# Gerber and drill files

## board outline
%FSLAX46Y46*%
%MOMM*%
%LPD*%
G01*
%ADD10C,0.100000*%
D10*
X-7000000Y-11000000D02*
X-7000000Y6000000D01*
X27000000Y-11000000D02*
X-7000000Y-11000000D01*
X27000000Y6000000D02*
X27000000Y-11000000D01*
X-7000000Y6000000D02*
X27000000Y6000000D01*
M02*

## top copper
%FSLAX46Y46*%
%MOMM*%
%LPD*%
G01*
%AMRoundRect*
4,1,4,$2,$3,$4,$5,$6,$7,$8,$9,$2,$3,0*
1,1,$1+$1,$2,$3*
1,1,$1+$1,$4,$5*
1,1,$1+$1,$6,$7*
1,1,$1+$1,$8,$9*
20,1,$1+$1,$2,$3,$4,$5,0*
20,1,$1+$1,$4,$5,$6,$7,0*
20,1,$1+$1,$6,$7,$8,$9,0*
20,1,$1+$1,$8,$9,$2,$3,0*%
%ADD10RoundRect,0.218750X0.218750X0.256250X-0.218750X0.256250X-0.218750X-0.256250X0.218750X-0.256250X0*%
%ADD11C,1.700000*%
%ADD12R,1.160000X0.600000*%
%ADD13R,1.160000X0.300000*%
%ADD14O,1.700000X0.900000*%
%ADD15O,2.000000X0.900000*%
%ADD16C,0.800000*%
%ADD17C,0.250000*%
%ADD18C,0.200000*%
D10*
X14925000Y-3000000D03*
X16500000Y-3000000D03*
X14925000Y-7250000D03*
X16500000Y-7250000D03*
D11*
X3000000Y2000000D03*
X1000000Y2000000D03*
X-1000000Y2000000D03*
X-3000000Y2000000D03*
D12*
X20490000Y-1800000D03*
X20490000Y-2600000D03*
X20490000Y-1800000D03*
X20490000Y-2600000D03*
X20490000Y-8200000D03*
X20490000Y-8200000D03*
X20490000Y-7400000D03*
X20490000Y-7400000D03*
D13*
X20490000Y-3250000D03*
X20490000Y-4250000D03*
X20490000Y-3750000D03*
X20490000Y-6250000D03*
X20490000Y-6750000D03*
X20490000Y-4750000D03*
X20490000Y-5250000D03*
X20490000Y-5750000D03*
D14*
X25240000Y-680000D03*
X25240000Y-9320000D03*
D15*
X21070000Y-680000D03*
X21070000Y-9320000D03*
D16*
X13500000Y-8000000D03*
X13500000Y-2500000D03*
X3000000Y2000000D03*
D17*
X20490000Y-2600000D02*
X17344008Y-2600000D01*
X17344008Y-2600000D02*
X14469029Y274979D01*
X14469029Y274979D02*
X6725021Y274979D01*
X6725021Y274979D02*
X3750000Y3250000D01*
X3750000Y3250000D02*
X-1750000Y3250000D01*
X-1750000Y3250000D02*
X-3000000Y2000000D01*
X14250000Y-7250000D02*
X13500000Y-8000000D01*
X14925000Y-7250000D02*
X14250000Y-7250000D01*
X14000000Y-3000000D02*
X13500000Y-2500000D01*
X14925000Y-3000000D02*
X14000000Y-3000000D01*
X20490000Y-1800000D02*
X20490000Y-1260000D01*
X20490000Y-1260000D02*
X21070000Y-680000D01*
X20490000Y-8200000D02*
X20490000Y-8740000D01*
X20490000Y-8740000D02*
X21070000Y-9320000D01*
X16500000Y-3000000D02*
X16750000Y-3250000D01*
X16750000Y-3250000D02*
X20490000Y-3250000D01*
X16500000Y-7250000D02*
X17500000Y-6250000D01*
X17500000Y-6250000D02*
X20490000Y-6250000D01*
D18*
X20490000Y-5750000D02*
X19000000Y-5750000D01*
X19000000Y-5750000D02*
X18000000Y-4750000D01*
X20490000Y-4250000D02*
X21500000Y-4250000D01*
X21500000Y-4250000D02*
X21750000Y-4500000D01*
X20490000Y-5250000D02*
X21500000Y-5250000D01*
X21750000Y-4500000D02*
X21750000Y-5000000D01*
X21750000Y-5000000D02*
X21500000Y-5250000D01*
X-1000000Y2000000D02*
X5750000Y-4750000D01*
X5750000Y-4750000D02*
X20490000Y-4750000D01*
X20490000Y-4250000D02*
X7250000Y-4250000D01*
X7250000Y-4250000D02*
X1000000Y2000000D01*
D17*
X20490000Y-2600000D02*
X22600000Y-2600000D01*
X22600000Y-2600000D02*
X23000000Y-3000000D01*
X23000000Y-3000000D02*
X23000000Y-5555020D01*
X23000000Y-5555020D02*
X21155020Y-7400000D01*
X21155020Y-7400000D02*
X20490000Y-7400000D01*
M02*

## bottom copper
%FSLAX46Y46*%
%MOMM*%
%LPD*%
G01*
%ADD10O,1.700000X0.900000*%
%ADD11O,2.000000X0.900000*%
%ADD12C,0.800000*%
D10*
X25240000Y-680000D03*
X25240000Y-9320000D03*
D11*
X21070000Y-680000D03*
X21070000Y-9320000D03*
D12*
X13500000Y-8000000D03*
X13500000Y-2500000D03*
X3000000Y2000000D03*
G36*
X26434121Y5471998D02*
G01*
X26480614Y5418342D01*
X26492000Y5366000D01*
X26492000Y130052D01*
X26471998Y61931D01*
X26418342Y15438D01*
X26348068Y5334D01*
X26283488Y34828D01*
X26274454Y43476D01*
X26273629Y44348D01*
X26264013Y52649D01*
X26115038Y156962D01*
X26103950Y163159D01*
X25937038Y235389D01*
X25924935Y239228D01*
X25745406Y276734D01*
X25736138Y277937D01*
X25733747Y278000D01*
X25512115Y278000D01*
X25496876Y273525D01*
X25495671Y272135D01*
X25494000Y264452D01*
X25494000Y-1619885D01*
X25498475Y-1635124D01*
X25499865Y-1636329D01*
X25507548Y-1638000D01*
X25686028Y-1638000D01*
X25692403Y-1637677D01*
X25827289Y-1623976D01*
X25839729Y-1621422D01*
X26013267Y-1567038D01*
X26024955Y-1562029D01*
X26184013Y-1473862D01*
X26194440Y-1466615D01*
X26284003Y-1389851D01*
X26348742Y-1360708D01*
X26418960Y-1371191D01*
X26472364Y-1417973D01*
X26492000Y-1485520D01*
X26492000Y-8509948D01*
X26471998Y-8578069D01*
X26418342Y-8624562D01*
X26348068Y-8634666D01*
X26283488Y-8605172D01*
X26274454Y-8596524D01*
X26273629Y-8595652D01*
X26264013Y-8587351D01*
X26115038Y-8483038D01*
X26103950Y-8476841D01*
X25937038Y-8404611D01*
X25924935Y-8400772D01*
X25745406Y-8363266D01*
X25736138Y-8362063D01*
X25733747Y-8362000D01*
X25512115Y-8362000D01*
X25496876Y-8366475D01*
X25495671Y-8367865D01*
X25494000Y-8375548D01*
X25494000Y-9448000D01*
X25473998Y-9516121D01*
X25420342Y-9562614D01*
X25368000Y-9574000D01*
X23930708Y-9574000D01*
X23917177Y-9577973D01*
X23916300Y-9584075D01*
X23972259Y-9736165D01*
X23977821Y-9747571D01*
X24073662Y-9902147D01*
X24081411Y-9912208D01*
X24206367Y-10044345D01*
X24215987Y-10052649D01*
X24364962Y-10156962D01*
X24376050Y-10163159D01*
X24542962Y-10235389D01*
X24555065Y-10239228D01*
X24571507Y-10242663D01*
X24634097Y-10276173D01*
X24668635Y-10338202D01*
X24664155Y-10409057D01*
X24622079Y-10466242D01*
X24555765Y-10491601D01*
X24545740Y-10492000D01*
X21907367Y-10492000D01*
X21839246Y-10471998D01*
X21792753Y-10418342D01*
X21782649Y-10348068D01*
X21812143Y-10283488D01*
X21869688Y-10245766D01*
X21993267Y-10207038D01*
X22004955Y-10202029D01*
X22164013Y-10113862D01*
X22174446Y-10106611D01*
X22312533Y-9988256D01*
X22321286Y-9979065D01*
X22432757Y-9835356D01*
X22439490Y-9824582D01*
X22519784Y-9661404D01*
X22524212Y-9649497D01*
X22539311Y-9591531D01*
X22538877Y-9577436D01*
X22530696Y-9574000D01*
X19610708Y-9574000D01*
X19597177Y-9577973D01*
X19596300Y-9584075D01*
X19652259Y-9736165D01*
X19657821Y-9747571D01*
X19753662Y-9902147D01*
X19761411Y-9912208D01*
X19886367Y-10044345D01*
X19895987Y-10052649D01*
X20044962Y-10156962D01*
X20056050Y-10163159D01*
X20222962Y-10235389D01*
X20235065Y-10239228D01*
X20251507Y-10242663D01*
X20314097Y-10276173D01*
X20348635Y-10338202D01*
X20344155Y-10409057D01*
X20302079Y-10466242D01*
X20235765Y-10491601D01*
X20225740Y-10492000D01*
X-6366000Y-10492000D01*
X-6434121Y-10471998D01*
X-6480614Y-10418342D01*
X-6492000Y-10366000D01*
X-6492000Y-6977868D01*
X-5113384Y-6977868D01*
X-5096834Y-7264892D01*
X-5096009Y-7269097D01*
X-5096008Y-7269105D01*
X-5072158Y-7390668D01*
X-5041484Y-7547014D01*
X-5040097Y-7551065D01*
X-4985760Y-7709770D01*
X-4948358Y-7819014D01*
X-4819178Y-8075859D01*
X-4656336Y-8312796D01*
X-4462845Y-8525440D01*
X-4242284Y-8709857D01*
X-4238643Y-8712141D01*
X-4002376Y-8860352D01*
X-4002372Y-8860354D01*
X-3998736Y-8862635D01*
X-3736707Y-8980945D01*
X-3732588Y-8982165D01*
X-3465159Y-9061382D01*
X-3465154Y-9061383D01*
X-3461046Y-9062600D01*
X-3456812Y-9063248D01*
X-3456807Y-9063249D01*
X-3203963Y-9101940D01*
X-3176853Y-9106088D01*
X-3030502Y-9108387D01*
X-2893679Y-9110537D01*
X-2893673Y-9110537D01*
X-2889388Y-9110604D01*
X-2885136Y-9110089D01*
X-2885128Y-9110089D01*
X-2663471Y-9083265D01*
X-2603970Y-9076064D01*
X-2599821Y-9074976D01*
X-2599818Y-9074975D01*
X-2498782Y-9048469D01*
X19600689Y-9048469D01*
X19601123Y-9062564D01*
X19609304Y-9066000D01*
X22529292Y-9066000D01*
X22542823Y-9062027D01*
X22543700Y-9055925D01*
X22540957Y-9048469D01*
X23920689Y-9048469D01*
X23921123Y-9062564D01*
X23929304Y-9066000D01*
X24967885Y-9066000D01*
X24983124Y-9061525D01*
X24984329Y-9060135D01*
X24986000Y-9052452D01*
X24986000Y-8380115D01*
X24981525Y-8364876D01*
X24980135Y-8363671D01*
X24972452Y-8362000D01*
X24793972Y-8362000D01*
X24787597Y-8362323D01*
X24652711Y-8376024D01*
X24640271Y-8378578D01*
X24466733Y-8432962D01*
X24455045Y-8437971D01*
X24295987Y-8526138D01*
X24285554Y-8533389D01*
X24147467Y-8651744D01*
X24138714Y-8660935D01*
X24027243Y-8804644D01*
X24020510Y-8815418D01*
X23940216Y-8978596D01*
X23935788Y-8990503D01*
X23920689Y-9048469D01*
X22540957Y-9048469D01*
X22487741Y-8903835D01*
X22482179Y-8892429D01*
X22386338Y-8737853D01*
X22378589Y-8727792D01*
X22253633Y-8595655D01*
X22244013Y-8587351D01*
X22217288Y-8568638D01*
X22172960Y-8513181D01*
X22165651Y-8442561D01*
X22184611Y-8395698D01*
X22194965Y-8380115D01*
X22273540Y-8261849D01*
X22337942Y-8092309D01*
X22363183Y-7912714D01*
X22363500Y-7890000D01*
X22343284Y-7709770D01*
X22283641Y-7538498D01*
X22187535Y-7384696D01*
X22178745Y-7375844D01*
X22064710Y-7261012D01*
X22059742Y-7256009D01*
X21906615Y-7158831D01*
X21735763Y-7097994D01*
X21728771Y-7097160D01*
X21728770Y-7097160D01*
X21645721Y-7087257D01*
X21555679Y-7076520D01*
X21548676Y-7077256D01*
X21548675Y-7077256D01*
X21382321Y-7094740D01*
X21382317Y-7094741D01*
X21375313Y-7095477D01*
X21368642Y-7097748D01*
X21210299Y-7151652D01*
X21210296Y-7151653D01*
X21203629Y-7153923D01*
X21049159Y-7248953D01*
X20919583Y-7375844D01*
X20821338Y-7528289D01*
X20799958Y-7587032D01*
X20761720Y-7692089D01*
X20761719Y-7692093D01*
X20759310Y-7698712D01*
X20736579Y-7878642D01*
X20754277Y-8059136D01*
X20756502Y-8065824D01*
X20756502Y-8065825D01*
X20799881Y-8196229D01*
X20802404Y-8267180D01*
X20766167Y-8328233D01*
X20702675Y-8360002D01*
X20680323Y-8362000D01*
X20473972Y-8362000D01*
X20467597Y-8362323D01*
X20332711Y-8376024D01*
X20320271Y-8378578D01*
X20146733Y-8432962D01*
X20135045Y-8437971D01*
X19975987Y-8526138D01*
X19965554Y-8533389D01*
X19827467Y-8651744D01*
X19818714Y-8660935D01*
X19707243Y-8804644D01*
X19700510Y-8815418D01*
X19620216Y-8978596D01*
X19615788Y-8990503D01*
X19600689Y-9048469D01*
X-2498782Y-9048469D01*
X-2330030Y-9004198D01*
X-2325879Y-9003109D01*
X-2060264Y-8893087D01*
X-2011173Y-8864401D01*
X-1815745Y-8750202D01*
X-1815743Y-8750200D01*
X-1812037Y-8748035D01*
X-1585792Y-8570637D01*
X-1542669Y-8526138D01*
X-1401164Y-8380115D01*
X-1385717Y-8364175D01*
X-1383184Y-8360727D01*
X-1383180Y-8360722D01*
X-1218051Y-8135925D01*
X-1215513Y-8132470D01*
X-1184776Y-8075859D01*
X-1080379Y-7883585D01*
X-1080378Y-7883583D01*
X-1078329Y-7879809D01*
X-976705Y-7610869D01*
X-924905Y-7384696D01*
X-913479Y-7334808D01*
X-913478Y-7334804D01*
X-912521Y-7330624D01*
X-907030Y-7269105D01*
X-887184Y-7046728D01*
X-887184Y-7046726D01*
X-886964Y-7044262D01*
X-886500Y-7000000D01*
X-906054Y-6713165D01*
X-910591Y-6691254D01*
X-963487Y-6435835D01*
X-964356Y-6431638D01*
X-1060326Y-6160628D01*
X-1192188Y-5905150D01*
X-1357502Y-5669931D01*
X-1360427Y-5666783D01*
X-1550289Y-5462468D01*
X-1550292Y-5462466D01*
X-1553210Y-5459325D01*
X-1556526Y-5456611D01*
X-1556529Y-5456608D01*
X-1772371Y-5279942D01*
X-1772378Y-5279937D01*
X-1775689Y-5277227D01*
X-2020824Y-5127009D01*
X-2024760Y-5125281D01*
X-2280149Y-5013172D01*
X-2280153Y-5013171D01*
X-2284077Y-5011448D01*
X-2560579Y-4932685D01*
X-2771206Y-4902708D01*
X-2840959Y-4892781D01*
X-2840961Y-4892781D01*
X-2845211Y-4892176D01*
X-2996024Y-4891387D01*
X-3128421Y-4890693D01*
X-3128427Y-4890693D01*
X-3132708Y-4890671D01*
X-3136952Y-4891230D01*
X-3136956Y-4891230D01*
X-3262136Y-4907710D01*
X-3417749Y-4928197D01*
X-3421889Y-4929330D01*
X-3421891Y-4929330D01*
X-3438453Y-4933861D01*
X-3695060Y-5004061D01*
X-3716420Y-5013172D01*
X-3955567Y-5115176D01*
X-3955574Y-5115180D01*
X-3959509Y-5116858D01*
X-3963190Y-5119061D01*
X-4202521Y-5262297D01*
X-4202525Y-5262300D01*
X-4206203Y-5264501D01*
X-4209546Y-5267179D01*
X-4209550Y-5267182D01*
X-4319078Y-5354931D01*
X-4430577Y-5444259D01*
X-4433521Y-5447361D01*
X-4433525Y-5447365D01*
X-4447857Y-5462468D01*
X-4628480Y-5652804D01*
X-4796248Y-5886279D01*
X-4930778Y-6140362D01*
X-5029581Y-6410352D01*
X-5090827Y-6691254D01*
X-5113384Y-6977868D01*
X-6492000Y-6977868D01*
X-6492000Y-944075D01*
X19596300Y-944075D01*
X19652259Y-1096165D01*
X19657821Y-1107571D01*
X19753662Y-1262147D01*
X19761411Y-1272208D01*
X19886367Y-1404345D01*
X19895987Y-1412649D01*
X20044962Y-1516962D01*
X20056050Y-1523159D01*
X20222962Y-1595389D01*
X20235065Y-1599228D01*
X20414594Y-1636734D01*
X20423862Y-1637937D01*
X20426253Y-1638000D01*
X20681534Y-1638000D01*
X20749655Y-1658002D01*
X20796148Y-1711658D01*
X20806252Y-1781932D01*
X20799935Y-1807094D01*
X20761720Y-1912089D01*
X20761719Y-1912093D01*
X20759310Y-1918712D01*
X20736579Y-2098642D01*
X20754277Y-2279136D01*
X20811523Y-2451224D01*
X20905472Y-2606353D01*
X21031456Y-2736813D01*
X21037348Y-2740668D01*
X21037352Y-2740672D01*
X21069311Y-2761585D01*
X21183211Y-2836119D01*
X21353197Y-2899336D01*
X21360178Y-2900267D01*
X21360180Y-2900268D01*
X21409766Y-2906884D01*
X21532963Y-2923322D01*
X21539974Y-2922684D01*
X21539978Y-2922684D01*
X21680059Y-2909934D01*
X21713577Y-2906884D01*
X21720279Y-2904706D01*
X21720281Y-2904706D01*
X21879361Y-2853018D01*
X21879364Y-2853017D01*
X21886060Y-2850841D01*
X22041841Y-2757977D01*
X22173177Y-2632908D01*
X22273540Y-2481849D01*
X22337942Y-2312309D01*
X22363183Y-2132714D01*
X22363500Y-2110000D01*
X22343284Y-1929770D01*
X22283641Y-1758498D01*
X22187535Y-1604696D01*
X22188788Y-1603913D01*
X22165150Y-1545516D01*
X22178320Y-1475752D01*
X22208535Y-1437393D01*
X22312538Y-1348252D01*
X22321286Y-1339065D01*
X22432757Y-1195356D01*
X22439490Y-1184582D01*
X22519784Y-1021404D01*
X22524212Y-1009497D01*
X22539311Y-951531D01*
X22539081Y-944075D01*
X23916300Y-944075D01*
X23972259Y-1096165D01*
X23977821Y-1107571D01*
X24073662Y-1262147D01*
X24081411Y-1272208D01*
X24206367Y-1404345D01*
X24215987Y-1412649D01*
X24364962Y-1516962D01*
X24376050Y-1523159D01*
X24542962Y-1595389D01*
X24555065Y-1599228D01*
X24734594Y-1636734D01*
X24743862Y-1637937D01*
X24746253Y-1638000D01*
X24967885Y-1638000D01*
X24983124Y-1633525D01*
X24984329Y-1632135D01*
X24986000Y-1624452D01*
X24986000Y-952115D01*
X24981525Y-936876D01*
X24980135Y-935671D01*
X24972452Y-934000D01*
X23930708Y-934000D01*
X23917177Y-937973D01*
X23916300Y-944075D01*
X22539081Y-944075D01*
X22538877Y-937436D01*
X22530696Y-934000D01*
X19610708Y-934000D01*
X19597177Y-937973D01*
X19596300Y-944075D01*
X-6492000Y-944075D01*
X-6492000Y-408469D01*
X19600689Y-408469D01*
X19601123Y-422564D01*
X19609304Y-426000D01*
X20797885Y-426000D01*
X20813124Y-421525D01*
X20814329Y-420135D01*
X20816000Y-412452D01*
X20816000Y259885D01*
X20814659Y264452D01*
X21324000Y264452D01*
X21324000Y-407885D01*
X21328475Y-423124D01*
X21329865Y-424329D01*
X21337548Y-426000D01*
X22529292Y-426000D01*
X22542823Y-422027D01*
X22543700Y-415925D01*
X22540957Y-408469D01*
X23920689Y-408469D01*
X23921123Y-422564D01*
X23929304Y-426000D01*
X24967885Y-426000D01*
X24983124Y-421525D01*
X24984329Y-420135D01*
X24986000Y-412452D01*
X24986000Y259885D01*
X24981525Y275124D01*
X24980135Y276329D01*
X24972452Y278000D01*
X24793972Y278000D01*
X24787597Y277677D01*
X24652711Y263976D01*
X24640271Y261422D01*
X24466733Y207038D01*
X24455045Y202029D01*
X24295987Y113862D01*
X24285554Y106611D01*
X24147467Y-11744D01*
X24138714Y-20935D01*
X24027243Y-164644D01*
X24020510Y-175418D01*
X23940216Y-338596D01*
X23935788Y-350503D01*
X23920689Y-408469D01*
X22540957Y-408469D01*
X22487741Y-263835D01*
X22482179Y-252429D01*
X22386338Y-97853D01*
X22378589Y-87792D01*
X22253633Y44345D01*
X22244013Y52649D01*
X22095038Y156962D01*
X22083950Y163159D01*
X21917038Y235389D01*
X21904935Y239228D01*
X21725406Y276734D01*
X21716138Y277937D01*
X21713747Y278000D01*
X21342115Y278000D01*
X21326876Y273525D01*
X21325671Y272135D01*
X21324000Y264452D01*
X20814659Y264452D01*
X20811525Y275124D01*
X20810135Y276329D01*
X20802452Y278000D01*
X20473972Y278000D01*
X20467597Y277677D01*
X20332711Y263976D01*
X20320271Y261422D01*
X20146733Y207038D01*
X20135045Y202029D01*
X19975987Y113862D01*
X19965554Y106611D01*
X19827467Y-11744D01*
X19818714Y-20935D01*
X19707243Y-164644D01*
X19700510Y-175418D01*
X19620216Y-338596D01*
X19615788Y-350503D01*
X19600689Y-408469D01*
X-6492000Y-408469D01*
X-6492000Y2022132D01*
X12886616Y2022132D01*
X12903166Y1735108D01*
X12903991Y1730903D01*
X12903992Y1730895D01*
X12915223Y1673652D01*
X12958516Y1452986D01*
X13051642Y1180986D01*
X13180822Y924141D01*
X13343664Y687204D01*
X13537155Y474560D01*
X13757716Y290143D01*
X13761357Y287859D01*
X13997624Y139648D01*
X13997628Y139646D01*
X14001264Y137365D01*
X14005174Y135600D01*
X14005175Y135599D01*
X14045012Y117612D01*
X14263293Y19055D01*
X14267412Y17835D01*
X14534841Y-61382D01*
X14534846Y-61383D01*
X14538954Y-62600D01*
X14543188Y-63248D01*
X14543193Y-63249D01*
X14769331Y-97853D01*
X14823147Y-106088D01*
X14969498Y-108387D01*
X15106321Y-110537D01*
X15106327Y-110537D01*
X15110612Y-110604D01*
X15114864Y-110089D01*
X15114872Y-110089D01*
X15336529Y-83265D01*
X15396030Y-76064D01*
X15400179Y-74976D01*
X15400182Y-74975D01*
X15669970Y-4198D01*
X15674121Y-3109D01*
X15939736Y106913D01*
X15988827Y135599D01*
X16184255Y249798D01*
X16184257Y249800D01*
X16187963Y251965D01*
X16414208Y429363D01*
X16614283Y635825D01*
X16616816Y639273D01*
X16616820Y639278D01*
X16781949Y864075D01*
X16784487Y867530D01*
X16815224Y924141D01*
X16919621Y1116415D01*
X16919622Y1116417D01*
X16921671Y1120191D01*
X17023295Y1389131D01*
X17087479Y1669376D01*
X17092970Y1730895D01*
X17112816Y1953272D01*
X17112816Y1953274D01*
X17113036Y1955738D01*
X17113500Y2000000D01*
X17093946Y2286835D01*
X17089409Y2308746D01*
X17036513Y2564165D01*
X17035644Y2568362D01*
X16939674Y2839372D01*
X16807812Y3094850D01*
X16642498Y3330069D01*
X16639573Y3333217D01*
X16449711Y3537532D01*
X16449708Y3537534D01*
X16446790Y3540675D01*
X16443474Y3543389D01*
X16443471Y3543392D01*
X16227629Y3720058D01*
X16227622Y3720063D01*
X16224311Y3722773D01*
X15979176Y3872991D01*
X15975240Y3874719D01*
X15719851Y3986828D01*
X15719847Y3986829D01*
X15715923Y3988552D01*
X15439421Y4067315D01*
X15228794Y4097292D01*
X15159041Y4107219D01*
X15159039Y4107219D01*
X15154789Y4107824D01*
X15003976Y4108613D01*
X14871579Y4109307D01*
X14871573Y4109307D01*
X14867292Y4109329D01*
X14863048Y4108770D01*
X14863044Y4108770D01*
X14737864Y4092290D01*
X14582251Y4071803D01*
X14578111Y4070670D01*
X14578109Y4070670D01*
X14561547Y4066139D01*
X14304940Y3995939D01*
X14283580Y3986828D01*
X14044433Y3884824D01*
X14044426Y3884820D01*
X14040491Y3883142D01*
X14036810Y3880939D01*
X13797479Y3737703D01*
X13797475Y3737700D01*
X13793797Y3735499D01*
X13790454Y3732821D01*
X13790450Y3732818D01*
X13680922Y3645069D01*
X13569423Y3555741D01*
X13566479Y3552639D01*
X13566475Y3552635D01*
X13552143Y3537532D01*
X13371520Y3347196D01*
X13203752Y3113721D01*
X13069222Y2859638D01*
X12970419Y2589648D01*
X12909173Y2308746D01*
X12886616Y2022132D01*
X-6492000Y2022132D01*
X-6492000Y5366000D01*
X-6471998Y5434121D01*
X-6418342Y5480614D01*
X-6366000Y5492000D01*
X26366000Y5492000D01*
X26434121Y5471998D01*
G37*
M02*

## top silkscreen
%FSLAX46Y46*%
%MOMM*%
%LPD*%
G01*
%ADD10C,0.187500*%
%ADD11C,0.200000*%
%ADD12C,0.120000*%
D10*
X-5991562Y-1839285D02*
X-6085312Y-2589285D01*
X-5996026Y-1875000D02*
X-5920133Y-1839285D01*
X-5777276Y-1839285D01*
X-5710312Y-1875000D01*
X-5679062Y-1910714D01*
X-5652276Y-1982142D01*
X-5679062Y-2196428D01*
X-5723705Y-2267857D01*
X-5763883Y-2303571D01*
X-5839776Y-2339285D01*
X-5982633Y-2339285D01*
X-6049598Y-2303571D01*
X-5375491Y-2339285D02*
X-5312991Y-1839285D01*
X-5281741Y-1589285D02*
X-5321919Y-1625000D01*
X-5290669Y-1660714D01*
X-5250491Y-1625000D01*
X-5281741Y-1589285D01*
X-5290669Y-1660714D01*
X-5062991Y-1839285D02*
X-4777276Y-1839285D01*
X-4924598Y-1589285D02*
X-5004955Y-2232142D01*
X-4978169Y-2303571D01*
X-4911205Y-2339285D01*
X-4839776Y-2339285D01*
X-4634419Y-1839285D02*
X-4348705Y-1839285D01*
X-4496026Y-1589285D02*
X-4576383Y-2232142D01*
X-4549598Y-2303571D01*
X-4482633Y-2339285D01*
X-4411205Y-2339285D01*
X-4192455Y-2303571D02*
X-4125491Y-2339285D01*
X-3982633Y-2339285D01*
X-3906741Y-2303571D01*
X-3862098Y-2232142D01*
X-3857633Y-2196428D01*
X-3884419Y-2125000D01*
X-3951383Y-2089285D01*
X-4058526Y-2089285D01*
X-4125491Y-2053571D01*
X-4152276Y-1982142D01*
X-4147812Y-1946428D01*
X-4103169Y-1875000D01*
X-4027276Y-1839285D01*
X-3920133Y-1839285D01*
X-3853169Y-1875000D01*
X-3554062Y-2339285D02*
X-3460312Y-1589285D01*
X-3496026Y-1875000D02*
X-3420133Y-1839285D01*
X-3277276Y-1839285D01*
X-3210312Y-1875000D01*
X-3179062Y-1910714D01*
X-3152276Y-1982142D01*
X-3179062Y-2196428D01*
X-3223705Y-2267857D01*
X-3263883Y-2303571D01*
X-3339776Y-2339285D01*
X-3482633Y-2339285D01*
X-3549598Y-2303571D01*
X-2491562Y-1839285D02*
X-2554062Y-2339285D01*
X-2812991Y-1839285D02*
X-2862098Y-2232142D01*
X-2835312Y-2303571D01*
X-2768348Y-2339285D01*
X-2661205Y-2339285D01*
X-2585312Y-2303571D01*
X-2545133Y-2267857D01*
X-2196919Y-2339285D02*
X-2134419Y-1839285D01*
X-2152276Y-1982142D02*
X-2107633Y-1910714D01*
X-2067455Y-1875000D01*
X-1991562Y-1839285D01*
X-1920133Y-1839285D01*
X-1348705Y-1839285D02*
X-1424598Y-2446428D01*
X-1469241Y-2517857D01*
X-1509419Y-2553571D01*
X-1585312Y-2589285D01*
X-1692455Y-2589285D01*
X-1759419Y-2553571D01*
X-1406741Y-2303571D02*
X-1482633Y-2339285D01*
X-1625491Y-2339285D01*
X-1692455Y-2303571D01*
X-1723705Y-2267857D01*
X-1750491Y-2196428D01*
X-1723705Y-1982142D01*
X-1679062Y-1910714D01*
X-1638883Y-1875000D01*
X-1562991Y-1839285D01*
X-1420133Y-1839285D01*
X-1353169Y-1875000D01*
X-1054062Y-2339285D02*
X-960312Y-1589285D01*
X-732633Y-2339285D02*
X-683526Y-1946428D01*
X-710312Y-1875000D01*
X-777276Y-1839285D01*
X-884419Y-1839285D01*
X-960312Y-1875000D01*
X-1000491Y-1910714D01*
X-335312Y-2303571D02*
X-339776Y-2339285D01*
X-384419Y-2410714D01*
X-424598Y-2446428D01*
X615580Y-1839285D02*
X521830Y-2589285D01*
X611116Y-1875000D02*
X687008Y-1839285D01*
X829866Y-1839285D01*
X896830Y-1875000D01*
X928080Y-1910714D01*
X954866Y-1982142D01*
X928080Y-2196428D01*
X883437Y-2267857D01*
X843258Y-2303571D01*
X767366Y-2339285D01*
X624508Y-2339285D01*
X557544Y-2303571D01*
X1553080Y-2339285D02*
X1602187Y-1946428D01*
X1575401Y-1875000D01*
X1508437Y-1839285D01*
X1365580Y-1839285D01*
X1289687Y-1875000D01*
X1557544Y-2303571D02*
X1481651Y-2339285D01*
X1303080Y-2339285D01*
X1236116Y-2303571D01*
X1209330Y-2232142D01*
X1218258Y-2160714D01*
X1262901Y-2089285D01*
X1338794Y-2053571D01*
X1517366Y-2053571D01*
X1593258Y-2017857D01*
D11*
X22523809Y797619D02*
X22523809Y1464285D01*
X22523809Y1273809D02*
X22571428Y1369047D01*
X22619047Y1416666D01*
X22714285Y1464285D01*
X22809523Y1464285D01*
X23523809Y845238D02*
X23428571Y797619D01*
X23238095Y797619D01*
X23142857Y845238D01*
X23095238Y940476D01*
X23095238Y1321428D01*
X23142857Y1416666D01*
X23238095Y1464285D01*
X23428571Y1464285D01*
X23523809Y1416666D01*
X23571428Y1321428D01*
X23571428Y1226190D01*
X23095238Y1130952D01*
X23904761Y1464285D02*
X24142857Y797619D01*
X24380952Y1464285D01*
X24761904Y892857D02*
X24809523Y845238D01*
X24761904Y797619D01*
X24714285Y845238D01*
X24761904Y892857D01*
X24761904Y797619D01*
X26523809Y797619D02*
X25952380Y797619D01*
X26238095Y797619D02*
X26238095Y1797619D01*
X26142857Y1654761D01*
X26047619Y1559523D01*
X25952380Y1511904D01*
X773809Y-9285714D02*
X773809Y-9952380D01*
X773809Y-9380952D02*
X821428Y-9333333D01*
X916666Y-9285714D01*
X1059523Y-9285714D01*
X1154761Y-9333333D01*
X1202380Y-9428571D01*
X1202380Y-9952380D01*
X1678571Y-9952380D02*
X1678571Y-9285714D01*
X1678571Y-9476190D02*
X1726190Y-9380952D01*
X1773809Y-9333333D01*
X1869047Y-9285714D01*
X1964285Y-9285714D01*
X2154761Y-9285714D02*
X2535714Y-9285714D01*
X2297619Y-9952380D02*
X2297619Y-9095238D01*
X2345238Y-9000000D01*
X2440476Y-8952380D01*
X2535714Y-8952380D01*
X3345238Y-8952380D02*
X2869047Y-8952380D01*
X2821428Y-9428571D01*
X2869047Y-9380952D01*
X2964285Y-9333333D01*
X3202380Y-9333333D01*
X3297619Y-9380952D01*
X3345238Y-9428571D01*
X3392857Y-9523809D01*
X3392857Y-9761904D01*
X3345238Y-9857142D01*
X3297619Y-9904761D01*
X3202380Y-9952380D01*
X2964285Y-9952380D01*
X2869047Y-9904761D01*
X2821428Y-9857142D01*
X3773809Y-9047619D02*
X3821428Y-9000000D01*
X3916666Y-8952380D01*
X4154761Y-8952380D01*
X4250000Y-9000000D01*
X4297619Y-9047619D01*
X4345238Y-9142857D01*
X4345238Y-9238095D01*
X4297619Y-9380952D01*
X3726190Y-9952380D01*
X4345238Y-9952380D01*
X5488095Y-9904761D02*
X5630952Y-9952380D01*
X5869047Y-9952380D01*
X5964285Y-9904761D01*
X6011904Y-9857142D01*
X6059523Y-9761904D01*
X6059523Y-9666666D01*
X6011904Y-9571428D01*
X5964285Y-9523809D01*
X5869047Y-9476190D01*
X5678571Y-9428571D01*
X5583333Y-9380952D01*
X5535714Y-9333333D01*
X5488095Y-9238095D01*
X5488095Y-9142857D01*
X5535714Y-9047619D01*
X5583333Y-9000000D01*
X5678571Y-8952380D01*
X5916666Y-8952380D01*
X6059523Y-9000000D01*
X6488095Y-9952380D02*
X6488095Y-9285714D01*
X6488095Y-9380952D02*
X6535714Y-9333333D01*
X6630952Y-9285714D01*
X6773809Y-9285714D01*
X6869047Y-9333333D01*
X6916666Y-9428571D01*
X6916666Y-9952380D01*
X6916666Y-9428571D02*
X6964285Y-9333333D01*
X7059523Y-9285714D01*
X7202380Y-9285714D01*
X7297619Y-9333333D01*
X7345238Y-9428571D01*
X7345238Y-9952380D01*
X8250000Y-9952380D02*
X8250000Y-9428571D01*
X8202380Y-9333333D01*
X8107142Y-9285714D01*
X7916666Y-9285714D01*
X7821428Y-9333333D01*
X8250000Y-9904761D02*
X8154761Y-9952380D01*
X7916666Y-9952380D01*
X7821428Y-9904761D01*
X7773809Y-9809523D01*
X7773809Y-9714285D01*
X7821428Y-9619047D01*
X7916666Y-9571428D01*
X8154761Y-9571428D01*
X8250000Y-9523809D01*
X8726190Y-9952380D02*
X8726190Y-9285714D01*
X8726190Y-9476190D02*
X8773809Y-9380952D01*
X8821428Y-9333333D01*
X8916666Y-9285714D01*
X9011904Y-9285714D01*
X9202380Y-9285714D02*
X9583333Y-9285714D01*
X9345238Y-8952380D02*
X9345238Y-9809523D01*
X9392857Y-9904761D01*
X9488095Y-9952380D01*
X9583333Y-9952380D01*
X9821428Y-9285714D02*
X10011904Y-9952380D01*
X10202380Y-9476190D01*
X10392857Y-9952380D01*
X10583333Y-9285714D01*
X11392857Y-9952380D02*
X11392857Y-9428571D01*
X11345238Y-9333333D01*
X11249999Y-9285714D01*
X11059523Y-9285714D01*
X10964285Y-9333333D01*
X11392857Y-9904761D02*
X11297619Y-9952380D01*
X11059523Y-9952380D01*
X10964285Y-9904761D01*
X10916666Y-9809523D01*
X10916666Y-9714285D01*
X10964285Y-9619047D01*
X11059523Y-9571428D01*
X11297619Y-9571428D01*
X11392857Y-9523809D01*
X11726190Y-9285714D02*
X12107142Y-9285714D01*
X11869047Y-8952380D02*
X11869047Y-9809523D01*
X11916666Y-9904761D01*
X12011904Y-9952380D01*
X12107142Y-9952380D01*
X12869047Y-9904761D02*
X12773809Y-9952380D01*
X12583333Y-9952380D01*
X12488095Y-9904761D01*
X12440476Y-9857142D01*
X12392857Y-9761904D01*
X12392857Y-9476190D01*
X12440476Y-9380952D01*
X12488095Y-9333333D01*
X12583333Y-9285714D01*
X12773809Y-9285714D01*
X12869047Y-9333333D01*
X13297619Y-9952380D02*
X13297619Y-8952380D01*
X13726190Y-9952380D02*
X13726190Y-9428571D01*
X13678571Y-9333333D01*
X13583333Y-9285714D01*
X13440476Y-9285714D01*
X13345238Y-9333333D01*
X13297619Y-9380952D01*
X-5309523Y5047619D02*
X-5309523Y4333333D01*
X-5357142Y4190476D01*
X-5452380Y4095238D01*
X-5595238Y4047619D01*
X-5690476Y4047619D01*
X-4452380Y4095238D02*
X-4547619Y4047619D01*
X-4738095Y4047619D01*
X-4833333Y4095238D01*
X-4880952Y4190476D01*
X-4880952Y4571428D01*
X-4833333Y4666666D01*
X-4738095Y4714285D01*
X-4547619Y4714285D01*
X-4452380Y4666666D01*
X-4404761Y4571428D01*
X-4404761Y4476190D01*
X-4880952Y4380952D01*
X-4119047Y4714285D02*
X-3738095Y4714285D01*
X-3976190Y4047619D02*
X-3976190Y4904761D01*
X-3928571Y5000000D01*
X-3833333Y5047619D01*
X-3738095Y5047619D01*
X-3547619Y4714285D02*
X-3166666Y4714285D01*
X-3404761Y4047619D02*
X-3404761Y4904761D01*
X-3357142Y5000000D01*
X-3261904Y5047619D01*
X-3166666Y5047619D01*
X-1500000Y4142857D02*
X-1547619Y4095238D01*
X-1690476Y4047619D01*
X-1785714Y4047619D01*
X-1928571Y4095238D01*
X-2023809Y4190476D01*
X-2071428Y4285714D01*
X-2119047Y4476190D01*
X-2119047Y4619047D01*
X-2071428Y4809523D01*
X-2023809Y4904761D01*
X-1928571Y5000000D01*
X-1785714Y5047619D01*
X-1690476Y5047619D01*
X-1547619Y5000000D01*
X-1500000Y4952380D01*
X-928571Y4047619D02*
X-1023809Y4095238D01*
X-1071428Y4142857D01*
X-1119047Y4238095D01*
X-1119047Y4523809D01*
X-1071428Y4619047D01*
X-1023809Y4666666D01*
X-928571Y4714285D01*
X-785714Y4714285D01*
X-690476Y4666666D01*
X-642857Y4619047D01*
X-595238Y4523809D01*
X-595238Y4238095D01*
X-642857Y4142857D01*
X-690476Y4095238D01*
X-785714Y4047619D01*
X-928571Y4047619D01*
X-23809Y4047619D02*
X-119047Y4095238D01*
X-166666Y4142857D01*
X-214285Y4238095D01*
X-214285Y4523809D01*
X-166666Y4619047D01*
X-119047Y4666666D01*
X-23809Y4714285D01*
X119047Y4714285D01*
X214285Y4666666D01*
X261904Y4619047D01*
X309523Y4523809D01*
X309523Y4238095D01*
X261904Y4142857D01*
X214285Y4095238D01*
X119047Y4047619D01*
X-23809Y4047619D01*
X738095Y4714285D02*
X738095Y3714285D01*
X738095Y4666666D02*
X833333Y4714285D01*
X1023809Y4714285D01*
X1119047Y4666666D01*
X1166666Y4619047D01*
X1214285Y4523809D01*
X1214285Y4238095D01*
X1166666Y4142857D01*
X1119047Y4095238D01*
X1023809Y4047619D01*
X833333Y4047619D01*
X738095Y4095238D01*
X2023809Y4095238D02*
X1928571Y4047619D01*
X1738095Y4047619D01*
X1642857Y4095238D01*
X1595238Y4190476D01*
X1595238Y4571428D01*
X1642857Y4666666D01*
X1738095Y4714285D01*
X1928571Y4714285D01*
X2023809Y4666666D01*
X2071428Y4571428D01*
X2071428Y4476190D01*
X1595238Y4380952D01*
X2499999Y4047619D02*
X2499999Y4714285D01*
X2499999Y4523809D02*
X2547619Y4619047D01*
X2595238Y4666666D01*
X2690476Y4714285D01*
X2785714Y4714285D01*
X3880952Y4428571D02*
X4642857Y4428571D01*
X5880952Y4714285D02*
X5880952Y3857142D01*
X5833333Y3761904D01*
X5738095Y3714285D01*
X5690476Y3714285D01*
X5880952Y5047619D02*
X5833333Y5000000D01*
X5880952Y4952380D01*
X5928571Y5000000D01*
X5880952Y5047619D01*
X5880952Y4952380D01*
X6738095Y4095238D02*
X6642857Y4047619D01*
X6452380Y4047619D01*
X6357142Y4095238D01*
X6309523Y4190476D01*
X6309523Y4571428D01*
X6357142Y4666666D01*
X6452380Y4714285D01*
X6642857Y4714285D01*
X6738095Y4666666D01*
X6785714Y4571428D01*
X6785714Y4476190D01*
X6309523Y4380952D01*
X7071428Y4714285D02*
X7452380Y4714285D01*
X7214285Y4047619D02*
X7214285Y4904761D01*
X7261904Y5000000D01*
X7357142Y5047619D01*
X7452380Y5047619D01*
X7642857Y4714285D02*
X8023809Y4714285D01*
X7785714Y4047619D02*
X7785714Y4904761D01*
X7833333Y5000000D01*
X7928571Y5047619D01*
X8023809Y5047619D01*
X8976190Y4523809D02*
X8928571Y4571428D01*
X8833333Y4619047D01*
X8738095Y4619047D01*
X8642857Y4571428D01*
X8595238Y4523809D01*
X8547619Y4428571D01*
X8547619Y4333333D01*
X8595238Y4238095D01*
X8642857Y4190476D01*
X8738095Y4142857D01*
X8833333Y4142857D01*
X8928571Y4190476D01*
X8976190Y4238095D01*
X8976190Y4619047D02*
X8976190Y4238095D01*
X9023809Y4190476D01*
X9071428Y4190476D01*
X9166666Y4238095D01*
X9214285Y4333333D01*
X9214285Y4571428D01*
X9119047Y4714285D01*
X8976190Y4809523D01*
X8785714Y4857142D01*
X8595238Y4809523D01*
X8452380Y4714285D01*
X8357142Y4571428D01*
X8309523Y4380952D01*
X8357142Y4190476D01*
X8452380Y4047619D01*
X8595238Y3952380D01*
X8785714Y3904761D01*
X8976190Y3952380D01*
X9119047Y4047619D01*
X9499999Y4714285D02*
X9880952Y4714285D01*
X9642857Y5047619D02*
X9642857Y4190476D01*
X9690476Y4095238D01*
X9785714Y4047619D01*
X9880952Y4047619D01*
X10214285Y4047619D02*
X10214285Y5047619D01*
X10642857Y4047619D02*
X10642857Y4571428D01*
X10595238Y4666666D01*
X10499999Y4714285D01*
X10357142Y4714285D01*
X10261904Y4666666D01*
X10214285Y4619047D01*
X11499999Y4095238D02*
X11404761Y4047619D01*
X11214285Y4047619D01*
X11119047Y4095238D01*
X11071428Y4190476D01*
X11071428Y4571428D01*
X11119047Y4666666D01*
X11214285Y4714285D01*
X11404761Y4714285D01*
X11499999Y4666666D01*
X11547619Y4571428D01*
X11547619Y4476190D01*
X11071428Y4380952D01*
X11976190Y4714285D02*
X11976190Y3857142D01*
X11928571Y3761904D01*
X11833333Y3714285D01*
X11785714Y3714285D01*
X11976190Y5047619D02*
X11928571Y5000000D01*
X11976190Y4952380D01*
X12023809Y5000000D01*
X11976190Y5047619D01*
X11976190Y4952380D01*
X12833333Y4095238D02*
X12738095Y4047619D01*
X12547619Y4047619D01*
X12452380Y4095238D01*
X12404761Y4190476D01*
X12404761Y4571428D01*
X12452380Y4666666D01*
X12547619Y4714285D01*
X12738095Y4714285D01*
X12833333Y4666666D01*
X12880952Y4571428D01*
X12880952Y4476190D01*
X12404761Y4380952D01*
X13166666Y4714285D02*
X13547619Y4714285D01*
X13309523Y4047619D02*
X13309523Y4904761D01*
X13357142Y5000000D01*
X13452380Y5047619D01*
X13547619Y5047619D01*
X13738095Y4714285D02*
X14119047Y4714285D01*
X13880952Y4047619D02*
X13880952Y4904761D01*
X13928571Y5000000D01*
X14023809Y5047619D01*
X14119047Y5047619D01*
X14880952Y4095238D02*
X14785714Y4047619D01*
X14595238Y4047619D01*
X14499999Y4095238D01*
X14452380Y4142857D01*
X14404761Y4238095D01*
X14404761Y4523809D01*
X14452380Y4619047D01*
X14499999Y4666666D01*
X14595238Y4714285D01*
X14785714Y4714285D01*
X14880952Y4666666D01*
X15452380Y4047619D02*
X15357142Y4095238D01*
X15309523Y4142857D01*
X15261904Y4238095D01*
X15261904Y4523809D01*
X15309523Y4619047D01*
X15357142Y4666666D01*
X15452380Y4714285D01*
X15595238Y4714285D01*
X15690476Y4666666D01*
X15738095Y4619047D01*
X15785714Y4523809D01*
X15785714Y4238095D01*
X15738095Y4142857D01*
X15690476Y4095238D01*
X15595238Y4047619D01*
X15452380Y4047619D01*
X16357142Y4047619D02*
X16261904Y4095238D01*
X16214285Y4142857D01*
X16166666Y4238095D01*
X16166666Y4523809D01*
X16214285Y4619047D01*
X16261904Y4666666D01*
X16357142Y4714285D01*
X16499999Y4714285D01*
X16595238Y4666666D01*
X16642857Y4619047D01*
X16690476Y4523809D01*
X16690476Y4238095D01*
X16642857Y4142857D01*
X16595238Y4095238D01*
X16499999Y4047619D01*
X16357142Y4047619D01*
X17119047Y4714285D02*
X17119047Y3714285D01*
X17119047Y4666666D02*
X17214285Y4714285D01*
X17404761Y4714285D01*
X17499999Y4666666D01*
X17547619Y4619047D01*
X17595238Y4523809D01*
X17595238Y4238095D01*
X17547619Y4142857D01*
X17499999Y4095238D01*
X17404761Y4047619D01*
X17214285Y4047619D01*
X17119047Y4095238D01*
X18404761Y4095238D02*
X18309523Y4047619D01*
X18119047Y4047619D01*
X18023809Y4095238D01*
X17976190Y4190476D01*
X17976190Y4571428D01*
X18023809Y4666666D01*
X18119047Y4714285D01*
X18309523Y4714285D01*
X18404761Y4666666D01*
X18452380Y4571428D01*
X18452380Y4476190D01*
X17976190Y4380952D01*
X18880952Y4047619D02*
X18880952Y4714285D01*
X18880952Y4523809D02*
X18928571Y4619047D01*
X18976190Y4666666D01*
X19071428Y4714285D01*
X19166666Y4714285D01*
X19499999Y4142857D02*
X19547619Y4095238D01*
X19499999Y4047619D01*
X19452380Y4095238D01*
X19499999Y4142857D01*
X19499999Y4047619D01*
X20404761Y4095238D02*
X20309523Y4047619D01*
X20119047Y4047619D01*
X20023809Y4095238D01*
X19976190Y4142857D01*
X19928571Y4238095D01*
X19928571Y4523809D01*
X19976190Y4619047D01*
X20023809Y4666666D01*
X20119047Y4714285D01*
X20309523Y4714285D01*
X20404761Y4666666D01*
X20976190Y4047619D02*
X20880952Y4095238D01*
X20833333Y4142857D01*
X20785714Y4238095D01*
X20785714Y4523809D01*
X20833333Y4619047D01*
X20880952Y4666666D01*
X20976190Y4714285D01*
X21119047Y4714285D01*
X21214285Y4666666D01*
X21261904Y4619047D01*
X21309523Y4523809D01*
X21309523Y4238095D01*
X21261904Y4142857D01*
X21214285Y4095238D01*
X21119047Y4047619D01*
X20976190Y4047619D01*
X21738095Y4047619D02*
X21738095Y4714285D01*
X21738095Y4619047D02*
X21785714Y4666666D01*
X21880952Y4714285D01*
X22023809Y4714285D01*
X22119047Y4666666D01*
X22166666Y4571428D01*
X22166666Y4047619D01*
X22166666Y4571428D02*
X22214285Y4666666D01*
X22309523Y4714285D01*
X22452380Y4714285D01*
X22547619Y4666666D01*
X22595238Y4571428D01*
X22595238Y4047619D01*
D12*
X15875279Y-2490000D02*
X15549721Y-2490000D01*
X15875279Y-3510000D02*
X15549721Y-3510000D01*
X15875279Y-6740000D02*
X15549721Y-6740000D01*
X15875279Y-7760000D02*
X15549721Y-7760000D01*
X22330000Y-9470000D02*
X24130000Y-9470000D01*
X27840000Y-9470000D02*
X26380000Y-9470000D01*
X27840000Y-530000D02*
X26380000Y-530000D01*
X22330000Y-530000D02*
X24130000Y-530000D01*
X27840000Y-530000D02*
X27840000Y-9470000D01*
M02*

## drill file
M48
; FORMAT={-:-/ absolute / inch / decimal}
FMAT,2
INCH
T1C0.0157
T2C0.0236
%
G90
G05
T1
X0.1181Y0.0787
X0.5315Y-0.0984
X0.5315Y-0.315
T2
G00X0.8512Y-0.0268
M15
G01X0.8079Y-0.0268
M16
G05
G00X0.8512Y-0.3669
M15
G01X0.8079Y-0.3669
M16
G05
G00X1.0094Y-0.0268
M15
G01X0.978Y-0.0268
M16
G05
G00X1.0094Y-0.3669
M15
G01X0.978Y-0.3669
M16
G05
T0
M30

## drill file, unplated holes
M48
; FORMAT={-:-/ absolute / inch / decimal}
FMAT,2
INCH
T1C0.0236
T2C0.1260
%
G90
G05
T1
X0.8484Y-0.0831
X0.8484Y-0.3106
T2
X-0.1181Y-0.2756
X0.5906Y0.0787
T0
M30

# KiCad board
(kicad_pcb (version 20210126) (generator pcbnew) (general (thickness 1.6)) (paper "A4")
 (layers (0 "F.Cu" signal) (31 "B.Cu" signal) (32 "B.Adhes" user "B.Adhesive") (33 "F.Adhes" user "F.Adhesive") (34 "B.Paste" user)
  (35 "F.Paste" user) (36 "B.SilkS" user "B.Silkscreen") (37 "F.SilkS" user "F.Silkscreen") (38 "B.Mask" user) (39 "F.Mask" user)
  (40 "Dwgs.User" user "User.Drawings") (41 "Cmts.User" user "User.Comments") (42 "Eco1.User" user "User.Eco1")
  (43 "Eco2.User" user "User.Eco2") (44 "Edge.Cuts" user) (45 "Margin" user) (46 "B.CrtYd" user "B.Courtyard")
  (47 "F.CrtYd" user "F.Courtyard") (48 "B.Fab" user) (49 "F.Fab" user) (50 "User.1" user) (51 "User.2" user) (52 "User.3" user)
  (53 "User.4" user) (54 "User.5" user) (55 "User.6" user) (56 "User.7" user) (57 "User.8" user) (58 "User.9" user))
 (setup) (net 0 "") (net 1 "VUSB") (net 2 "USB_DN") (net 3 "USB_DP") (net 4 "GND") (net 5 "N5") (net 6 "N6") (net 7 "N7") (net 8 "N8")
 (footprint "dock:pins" (layer "F.Cu") (at 0 -2)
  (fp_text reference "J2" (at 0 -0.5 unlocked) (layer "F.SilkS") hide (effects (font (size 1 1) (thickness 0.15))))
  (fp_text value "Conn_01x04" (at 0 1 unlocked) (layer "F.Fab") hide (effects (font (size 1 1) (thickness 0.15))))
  (pad "1" smd circle (at -3 0) (locked) (size 1.7 1.7) (layers "F.Cu" "F.Paste" "F.Mask") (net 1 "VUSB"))
  (pad "2" smd circle (at -1 0) (locked) (size 1.7 1.7) (layers "F.Cu" "F.Paste" "F.Mask") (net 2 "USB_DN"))
  (pad "3" smd circle (at 1 0) (locked) (size 1.7 1.7) (layers "F.Cu" "F.Paste" "F.Mask") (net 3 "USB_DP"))
  (pad "4" smd circle (at 3 0) (locked) (size 1.7 1.7) (layers "F.Cu" "F.Paste" "F.Mask") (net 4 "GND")))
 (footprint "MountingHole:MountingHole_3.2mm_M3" (layer "F.Cu") (at -3 7)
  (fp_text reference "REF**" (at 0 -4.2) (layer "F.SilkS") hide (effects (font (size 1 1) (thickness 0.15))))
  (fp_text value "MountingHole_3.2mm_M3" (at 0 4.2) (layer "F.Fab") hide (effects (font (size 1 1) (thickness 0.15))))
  (pad "1" np_thru_hole circle (at 0 0) (locked) (size 3.2 3.2) (drill 3.2) (layers *.Cu *.Mask)))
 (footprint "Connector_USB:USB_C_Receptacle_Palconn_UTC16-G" (layer "F.Cu") (at 23 5 90)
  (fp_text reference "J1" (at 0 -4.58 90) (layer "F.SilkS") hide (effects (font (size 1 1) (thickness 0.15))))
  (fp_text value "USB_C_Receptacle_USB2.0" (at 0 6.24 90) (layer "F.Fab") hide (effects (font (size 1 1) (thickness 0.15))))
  (fp_line (start -4.47 -0.67) (end -4.47 1.13) (layer "F.SilkS") (width 0.12))
  (fp_line (start 4.47 4.84) (end -4.47 4.84) (layer "F.SilkS") (width 0.12))
  (fp_line (start -4.47 4.84) (end -4.47 3.38) (layer "F.SilkS") (width 0.12))
  (fp_line (start 4.47 4.84) (end 4.47 3.38) (layer "F.SilkS") (width 0.12))
  (fp_line (start 4.47 -0.67) (end 4.47 1.13) (layer "F.SilkS") (width 0.12))
  (pad "" np_thru_hole circle (at -2.89 -1.45 270) (locked) (size 0.6 0.6) (drill 0.6) (layers *.Cu *.Mask))
  (pad "" np_thru_hole circle (at 2.89 -1.45 270) (locked) (size 0.6 0.6) (drill 0.6) (layers *.Cu *.Mask))
  (pad "A1" smd rect (at -3.2 -2.51 90) (locked) (size 0.6 1.16) (layers "F.Cu" "F.Paste" "F.Mask") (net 4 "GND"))
  (pad "A4" smd rect (at -2.4 -2.51 90) (locked) (size 0.6 1.16) (layers "F.Cu" "F.Paste" "F.Mask") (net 1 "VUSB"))
  (pad "A5" smd rect (at -1.25 -2.51 270) (locked) (size 0.3 1.16) (layers "F.Cu" "F.Paste" "F.Mask") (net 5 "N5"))
  (pad "A6" smd rect (at -0.25 -2.51 270) (locked) (size 0.3 1.16) (layers "F.Cu" "F.Paste" "F.Mask") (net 3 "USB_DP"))
  (pad "A7" smd rect (at 0.25 -2.51 270) (locked) (size 0.3 1.16) (layers "F.Cu" "F.Paste" "F.Mask") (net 2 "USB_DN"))
  (pad "A8" smd rect (at 1.25 -2.51 270) (locked) (size 0.3 1.16) (layers "F.Cu" "F.Paste" "F.Mask") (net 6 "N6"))
  (pad "A9" smd rect (at 2.4 -2.51 90) (locked) (size 0.6 1.16) (layers "F.Cu" "F.Paste" "F.Mask") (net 1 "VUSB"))
  (pad "A12" smd rect (at 3.2 -2.51 90) (locked) (size 0.6 1.16) (layers "F.Cu" "F.Paste" "F.Mask") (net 4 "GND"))
  (pad "B1" smd rect (at 3.2 -2.51 90) (locked) (size 0.6 1.16) (layers "F.Cu" "F.Paste" "F.Mask") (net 4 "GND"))
  (pad "B4" smd rect (at 2.4 -2.51 90) (locked) (size 0.6 1.16) (layers "F.Cu" "F.Paste" "F.Mask") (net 1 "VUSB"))
  (pad "B5" smd rect (at 1.75 -2.51 270) (locked) (size 0.3 1.16) (layers "F.Cu" "F.Paste" "F.Mask") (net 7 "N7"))
  (pad "B6" smd rect (at 0.75 -2.51 270) (locked) (size 0.3 1.16) (layers "F.Cu" "F.Paste" "F.Mask") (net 3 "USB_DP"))
  (pad "B7" smd rect (at -0.75 -2.51 270) (locked) (size 0.3 1.16) (layers "F.Cu" "F.Paste" "F.Mask") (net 2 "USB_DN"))
  (pad "B8" smd rect (at -1.75 -2.51 270) (locked) (size 0.3 1.16) (layers "F.Cu" "F.Paste" "F.Mask") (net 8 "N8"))
  (pad "B9" smd rect (at -2.4 -2.51 90) (locked) (size 0.6 1.16) (layers "F.Cu" "F.Paste" "F.Mask") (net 1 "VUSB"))
  (pad "B12" smd rect (at -3.2 -2.51 90) (locked) (size 0.6 1.16) (layers "F.Cu" "F.Paste" "F.Mask") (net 4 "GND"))
  (pad "S1" thru_hole oval (at 4.32 -1.93 180) (locked) (size 2 0.9) (drill oval 1.7 0.6) (layers *.Cu *.Mask) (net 4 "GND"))
  (pad "S1" thru_hole oval (at -4.32 2.24 180) (locked) (size 1.7 0.9) (drill oval 1.4 0.6) (layers *.Cu *.Mask) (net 4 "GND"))
  (pad "S1" thru_hole oval (at 4.32 2.24 180) (locked) (size 1.7 0.9) (drill oval 1.4 0.6) (layers *.Cu *.Mask) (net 4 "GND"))
  (pad "S1" thru_hole oval (at -4.32 -1.93 180) (locked) (size 2 0.9) (drill oval 1.7 0.6) (layers *.Cu *.Mask) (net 4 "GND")))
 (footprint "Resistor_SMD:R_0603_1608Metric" (layer "F.Cu") (at 15.7125 3 180)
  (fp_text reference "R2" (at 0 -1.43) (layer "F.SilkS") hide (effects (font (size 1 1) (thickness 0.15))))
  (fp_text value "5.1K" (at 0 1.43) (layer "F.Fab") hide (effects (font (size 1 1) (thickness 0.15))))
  (fp_line (start -0.162779 -0.51) (end 0.162779 -0.51) (layer "F.SilkS") (width 0.12))
  (fp_line (start -0.162779 0.51) (end 0.162779 0.51) (layer "F.SilkS") (width 0.12))
  (pad "1" smd roundrect (at -0.7875 0 180) (locked) (size 0.875 0.95) (layers "F.Cu" "F.Paste" "F.Mask") (roundrect_rratio 0.25)
   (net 7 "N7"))
  (pad "2" smd roundrect (at 0.7875 0 180) (locked) (size 0.875 0.95) (layers "F.Cu" "F.Paste" "F.Mask") (roundrect_rratio 0.25)
   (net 4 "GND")))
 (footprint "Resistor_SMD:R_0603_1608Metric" (layer "F.Cu") (at 15.7125 7.25 180)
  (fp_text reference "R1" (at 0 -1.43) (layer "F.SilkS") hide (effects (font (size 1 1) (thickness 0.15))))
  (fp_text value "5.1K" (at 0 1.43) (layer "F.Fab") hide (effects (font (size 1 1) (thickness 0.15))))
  (fp_line (start -0.162779 0.51) (end 0.162779 0.51) (layer "F.SilkS") (width 0.12))
  (fp_line (start -0.162779 -0.51) (end 0.162779 -0.51) (layer "F.SilkS") (width 0.12))
  (pad "1" smd roundrect (at -0.7875 0 180) (locked) (size 0.875 0.95) (layers "F.Cu" "F.Paste" "F.Mask") (roundrect_rratio 0.25)
   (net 5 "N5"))
  (pad "2" smd roundrect (at 0.7875 0 180) (locked) (size 0.875 0.95) (layers "F.Cu" "F.Paste" "F.Mask") (roundrect_rratio 0.25)
   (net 4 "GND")))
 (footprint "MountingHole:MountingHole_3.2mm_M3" (layer "F.Cu") (at 15 -2)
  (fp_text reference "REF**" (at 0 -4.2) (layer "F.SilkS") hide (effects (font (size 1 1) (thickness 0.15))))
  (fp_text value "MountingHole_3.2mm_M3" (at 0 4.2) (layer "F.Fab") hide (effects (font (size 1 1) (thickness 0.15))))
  (pad "1" np_thru_hole circle (at 0 0) (locked) (size 3.2 3.2) (drill 3.2) (layers *.Cu *.Mask)))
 (gr_line (start 27 11) (end -7 11) (layer "Edge.Cuts") (width 0.1))
 (gr_line (start 27 -6) (end 27 11) (layer "Edge.Cuts") (width 0.1))
 (gr_line (start -7 -6) (end 27 -6) (layer "Edge.Cuts") (width 0.1))
 (gr_line (start -7 11) (end -7 -6) (layer "Edge.Cuts") (width 0.1))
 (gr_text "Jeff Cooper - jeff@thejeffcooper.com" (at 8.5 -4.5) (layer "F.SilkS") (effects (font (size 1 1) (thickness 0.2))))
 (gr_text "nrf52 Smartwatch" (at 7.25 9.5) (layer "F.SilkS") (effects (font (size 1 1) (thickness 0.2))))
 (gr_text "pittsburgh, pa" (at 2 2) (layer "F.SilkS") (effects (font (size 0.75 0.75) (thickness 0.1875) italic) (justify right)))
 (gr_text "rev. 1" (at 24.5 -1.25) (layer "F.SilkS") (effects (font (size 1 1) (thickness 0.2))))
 (segment (start 14.925 7.25) (end 14.25 7.25) (width 0.25) (layer "F.Cu") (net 4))
 (segment (start 14.925 3) (end 14 3) (width 0.25) (layer "F.Cu") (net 4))
 (segment (start 20.49 1.8) (end 20.49 1.26) (width 0.25) (layer "F.Cu") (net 4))
 (segment (start 14.25 7.25) (end 13.5 8) (width 0.25) (layer "F.Cu") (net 4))
 (segment (start 20.49 8.2) (end 20.49 8.74) (width 0.25) (layer "F.Cu") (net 4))
 (segment (start 14 3) (end 13.5 2.5) (width 0.25) (layer "F.Cu") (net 4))
 (segment (start 20.49 1.26) (end 21.07 0.68) (width 0.25) (layer "F.Cu") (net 4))
 (segment (start 20.49 8.74) (end 21.07 9.32) (width 0.25) (layer "F.Cu") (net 4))
 (via (at 13.5 2.5) (size 0.8) (drill 0.4) (layers "F.Cu" "B.Cu") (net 4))
 (via (at 13.5 8) (size 0.8) (drill 0.4) (layers "F.Cu" "B.Cu") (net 4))
 (via (at 3 -2) (size 0.8) (drill 0.4) (layers "F.Cu" "B.Cu") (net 4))
 (segment (start 3.75 -3.25) (end -1.75 -3.25) (width 0.25) (layer "F.Cu") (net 1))
 (segment (start 6.725021 -0.274979) (end 3.75 -3.25) (width 0.25) (layer "F.Cu") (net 1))
 (segment (start 22.6 2.6) (end 23 3) (width 0.25) (layer "F.Cu") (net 1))
 (segment (start 17.344008 2.6) (end 14.469029 -0.274979) (width 0.25) (layer "F.Cu") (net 1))
 (segment (start 14.469029 -0.274979) (end 6.725021 -0.274979) (width 0.25) (layer "F.Cu") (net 1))
 (segment (start -1.75 -3.25) (end -3 -2) (width 0.25) (layer "F.Cu") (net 1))
 (segment (start 20.49 2.6) (end 22.6 2.6) (width 0.25) (layer "F.Cu") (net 1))
 (segment (start 20.49 2.6) (end 17.344008 2.6) (width 0.25) (layer "F.Cu") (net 1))
 (segment (start 23 5.55502) (end 21.15502 7.4) (width 0.25) (layer "F.Cu") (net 1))
 (segment (start 21.15502 7.4) (end 20.49 7.4) (width 0.25) (layer "F.Cu") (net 1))
 (segment (start 23 3) (end 23 5.55502) (width 0.25) (layer "F.Cu") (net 1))
 (segment (start 16.5 3) (end 16.75 3.25) (width 0.25) (layer "F.Cu") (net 7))
 (segment (start 16.75 3.25) (end 20.49 3.25) (width 0.25) (layer "F.Cu") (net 7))
 (segment (start 20.49 4.25) (end 7.25 4.25) (width 0.2) (layer "F.Cu") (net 3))
 (segment (start 7.25 4.25) (end 1 -2) (width 0.2) (layer "F.Cu") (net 3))
 (segment (start 21.75 5) (end 21.5 5.25) (width 0.2) (layer "F.Cu") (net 3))
 (segment (start 20.49 5.25) (end 21.5 5.25) (width 0.2) (layer "F.Cu") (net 3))
 (segment (start 21.5 4.25) (end 21.75 4.5) (width 0.2) (layer "F.Cu") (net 3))
 (segment (start 21.75 4.5) (end 21.75 5) (width 0.2) (layer "F.Cu") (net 3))
 (segment (start 20.49 4.25) (end 21.5 4.25) (width 0.2) (layer "F.Cu") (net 3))
 (segment (start 17.5 6.25) (end 20.49 6.25) (width 0.25) (layer "F.Cu") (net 5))
 (segment (start 16.5 7.25) (end 17.5 6.25) (width 0.25) (layer "F.Cu") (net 5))
 (segment (start -1 -2) (end 5.75 4.75) (width 0.2) (layer "F.Cu") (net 2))
 (segment (start 5.75 4.75) (end 20.49 4.75) (width 0.2) (layer "F.Cu") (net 2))
 (segment (start 19 5.75) (end 18 4.75) (width 0.2) (layer "F.Cu") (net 2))
 (segment (start 20.49 5.75) (end 19 5.75) (width 0.2) (layer "F.Cu") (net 2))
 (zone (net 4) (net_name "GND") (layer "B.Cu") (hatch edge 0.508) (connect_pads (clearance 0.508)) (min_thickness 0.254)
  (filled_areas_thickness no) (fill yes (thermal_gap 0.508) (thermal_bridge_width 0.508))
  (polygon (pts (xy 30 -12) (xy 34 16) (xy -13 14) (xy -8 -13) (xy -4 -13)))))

